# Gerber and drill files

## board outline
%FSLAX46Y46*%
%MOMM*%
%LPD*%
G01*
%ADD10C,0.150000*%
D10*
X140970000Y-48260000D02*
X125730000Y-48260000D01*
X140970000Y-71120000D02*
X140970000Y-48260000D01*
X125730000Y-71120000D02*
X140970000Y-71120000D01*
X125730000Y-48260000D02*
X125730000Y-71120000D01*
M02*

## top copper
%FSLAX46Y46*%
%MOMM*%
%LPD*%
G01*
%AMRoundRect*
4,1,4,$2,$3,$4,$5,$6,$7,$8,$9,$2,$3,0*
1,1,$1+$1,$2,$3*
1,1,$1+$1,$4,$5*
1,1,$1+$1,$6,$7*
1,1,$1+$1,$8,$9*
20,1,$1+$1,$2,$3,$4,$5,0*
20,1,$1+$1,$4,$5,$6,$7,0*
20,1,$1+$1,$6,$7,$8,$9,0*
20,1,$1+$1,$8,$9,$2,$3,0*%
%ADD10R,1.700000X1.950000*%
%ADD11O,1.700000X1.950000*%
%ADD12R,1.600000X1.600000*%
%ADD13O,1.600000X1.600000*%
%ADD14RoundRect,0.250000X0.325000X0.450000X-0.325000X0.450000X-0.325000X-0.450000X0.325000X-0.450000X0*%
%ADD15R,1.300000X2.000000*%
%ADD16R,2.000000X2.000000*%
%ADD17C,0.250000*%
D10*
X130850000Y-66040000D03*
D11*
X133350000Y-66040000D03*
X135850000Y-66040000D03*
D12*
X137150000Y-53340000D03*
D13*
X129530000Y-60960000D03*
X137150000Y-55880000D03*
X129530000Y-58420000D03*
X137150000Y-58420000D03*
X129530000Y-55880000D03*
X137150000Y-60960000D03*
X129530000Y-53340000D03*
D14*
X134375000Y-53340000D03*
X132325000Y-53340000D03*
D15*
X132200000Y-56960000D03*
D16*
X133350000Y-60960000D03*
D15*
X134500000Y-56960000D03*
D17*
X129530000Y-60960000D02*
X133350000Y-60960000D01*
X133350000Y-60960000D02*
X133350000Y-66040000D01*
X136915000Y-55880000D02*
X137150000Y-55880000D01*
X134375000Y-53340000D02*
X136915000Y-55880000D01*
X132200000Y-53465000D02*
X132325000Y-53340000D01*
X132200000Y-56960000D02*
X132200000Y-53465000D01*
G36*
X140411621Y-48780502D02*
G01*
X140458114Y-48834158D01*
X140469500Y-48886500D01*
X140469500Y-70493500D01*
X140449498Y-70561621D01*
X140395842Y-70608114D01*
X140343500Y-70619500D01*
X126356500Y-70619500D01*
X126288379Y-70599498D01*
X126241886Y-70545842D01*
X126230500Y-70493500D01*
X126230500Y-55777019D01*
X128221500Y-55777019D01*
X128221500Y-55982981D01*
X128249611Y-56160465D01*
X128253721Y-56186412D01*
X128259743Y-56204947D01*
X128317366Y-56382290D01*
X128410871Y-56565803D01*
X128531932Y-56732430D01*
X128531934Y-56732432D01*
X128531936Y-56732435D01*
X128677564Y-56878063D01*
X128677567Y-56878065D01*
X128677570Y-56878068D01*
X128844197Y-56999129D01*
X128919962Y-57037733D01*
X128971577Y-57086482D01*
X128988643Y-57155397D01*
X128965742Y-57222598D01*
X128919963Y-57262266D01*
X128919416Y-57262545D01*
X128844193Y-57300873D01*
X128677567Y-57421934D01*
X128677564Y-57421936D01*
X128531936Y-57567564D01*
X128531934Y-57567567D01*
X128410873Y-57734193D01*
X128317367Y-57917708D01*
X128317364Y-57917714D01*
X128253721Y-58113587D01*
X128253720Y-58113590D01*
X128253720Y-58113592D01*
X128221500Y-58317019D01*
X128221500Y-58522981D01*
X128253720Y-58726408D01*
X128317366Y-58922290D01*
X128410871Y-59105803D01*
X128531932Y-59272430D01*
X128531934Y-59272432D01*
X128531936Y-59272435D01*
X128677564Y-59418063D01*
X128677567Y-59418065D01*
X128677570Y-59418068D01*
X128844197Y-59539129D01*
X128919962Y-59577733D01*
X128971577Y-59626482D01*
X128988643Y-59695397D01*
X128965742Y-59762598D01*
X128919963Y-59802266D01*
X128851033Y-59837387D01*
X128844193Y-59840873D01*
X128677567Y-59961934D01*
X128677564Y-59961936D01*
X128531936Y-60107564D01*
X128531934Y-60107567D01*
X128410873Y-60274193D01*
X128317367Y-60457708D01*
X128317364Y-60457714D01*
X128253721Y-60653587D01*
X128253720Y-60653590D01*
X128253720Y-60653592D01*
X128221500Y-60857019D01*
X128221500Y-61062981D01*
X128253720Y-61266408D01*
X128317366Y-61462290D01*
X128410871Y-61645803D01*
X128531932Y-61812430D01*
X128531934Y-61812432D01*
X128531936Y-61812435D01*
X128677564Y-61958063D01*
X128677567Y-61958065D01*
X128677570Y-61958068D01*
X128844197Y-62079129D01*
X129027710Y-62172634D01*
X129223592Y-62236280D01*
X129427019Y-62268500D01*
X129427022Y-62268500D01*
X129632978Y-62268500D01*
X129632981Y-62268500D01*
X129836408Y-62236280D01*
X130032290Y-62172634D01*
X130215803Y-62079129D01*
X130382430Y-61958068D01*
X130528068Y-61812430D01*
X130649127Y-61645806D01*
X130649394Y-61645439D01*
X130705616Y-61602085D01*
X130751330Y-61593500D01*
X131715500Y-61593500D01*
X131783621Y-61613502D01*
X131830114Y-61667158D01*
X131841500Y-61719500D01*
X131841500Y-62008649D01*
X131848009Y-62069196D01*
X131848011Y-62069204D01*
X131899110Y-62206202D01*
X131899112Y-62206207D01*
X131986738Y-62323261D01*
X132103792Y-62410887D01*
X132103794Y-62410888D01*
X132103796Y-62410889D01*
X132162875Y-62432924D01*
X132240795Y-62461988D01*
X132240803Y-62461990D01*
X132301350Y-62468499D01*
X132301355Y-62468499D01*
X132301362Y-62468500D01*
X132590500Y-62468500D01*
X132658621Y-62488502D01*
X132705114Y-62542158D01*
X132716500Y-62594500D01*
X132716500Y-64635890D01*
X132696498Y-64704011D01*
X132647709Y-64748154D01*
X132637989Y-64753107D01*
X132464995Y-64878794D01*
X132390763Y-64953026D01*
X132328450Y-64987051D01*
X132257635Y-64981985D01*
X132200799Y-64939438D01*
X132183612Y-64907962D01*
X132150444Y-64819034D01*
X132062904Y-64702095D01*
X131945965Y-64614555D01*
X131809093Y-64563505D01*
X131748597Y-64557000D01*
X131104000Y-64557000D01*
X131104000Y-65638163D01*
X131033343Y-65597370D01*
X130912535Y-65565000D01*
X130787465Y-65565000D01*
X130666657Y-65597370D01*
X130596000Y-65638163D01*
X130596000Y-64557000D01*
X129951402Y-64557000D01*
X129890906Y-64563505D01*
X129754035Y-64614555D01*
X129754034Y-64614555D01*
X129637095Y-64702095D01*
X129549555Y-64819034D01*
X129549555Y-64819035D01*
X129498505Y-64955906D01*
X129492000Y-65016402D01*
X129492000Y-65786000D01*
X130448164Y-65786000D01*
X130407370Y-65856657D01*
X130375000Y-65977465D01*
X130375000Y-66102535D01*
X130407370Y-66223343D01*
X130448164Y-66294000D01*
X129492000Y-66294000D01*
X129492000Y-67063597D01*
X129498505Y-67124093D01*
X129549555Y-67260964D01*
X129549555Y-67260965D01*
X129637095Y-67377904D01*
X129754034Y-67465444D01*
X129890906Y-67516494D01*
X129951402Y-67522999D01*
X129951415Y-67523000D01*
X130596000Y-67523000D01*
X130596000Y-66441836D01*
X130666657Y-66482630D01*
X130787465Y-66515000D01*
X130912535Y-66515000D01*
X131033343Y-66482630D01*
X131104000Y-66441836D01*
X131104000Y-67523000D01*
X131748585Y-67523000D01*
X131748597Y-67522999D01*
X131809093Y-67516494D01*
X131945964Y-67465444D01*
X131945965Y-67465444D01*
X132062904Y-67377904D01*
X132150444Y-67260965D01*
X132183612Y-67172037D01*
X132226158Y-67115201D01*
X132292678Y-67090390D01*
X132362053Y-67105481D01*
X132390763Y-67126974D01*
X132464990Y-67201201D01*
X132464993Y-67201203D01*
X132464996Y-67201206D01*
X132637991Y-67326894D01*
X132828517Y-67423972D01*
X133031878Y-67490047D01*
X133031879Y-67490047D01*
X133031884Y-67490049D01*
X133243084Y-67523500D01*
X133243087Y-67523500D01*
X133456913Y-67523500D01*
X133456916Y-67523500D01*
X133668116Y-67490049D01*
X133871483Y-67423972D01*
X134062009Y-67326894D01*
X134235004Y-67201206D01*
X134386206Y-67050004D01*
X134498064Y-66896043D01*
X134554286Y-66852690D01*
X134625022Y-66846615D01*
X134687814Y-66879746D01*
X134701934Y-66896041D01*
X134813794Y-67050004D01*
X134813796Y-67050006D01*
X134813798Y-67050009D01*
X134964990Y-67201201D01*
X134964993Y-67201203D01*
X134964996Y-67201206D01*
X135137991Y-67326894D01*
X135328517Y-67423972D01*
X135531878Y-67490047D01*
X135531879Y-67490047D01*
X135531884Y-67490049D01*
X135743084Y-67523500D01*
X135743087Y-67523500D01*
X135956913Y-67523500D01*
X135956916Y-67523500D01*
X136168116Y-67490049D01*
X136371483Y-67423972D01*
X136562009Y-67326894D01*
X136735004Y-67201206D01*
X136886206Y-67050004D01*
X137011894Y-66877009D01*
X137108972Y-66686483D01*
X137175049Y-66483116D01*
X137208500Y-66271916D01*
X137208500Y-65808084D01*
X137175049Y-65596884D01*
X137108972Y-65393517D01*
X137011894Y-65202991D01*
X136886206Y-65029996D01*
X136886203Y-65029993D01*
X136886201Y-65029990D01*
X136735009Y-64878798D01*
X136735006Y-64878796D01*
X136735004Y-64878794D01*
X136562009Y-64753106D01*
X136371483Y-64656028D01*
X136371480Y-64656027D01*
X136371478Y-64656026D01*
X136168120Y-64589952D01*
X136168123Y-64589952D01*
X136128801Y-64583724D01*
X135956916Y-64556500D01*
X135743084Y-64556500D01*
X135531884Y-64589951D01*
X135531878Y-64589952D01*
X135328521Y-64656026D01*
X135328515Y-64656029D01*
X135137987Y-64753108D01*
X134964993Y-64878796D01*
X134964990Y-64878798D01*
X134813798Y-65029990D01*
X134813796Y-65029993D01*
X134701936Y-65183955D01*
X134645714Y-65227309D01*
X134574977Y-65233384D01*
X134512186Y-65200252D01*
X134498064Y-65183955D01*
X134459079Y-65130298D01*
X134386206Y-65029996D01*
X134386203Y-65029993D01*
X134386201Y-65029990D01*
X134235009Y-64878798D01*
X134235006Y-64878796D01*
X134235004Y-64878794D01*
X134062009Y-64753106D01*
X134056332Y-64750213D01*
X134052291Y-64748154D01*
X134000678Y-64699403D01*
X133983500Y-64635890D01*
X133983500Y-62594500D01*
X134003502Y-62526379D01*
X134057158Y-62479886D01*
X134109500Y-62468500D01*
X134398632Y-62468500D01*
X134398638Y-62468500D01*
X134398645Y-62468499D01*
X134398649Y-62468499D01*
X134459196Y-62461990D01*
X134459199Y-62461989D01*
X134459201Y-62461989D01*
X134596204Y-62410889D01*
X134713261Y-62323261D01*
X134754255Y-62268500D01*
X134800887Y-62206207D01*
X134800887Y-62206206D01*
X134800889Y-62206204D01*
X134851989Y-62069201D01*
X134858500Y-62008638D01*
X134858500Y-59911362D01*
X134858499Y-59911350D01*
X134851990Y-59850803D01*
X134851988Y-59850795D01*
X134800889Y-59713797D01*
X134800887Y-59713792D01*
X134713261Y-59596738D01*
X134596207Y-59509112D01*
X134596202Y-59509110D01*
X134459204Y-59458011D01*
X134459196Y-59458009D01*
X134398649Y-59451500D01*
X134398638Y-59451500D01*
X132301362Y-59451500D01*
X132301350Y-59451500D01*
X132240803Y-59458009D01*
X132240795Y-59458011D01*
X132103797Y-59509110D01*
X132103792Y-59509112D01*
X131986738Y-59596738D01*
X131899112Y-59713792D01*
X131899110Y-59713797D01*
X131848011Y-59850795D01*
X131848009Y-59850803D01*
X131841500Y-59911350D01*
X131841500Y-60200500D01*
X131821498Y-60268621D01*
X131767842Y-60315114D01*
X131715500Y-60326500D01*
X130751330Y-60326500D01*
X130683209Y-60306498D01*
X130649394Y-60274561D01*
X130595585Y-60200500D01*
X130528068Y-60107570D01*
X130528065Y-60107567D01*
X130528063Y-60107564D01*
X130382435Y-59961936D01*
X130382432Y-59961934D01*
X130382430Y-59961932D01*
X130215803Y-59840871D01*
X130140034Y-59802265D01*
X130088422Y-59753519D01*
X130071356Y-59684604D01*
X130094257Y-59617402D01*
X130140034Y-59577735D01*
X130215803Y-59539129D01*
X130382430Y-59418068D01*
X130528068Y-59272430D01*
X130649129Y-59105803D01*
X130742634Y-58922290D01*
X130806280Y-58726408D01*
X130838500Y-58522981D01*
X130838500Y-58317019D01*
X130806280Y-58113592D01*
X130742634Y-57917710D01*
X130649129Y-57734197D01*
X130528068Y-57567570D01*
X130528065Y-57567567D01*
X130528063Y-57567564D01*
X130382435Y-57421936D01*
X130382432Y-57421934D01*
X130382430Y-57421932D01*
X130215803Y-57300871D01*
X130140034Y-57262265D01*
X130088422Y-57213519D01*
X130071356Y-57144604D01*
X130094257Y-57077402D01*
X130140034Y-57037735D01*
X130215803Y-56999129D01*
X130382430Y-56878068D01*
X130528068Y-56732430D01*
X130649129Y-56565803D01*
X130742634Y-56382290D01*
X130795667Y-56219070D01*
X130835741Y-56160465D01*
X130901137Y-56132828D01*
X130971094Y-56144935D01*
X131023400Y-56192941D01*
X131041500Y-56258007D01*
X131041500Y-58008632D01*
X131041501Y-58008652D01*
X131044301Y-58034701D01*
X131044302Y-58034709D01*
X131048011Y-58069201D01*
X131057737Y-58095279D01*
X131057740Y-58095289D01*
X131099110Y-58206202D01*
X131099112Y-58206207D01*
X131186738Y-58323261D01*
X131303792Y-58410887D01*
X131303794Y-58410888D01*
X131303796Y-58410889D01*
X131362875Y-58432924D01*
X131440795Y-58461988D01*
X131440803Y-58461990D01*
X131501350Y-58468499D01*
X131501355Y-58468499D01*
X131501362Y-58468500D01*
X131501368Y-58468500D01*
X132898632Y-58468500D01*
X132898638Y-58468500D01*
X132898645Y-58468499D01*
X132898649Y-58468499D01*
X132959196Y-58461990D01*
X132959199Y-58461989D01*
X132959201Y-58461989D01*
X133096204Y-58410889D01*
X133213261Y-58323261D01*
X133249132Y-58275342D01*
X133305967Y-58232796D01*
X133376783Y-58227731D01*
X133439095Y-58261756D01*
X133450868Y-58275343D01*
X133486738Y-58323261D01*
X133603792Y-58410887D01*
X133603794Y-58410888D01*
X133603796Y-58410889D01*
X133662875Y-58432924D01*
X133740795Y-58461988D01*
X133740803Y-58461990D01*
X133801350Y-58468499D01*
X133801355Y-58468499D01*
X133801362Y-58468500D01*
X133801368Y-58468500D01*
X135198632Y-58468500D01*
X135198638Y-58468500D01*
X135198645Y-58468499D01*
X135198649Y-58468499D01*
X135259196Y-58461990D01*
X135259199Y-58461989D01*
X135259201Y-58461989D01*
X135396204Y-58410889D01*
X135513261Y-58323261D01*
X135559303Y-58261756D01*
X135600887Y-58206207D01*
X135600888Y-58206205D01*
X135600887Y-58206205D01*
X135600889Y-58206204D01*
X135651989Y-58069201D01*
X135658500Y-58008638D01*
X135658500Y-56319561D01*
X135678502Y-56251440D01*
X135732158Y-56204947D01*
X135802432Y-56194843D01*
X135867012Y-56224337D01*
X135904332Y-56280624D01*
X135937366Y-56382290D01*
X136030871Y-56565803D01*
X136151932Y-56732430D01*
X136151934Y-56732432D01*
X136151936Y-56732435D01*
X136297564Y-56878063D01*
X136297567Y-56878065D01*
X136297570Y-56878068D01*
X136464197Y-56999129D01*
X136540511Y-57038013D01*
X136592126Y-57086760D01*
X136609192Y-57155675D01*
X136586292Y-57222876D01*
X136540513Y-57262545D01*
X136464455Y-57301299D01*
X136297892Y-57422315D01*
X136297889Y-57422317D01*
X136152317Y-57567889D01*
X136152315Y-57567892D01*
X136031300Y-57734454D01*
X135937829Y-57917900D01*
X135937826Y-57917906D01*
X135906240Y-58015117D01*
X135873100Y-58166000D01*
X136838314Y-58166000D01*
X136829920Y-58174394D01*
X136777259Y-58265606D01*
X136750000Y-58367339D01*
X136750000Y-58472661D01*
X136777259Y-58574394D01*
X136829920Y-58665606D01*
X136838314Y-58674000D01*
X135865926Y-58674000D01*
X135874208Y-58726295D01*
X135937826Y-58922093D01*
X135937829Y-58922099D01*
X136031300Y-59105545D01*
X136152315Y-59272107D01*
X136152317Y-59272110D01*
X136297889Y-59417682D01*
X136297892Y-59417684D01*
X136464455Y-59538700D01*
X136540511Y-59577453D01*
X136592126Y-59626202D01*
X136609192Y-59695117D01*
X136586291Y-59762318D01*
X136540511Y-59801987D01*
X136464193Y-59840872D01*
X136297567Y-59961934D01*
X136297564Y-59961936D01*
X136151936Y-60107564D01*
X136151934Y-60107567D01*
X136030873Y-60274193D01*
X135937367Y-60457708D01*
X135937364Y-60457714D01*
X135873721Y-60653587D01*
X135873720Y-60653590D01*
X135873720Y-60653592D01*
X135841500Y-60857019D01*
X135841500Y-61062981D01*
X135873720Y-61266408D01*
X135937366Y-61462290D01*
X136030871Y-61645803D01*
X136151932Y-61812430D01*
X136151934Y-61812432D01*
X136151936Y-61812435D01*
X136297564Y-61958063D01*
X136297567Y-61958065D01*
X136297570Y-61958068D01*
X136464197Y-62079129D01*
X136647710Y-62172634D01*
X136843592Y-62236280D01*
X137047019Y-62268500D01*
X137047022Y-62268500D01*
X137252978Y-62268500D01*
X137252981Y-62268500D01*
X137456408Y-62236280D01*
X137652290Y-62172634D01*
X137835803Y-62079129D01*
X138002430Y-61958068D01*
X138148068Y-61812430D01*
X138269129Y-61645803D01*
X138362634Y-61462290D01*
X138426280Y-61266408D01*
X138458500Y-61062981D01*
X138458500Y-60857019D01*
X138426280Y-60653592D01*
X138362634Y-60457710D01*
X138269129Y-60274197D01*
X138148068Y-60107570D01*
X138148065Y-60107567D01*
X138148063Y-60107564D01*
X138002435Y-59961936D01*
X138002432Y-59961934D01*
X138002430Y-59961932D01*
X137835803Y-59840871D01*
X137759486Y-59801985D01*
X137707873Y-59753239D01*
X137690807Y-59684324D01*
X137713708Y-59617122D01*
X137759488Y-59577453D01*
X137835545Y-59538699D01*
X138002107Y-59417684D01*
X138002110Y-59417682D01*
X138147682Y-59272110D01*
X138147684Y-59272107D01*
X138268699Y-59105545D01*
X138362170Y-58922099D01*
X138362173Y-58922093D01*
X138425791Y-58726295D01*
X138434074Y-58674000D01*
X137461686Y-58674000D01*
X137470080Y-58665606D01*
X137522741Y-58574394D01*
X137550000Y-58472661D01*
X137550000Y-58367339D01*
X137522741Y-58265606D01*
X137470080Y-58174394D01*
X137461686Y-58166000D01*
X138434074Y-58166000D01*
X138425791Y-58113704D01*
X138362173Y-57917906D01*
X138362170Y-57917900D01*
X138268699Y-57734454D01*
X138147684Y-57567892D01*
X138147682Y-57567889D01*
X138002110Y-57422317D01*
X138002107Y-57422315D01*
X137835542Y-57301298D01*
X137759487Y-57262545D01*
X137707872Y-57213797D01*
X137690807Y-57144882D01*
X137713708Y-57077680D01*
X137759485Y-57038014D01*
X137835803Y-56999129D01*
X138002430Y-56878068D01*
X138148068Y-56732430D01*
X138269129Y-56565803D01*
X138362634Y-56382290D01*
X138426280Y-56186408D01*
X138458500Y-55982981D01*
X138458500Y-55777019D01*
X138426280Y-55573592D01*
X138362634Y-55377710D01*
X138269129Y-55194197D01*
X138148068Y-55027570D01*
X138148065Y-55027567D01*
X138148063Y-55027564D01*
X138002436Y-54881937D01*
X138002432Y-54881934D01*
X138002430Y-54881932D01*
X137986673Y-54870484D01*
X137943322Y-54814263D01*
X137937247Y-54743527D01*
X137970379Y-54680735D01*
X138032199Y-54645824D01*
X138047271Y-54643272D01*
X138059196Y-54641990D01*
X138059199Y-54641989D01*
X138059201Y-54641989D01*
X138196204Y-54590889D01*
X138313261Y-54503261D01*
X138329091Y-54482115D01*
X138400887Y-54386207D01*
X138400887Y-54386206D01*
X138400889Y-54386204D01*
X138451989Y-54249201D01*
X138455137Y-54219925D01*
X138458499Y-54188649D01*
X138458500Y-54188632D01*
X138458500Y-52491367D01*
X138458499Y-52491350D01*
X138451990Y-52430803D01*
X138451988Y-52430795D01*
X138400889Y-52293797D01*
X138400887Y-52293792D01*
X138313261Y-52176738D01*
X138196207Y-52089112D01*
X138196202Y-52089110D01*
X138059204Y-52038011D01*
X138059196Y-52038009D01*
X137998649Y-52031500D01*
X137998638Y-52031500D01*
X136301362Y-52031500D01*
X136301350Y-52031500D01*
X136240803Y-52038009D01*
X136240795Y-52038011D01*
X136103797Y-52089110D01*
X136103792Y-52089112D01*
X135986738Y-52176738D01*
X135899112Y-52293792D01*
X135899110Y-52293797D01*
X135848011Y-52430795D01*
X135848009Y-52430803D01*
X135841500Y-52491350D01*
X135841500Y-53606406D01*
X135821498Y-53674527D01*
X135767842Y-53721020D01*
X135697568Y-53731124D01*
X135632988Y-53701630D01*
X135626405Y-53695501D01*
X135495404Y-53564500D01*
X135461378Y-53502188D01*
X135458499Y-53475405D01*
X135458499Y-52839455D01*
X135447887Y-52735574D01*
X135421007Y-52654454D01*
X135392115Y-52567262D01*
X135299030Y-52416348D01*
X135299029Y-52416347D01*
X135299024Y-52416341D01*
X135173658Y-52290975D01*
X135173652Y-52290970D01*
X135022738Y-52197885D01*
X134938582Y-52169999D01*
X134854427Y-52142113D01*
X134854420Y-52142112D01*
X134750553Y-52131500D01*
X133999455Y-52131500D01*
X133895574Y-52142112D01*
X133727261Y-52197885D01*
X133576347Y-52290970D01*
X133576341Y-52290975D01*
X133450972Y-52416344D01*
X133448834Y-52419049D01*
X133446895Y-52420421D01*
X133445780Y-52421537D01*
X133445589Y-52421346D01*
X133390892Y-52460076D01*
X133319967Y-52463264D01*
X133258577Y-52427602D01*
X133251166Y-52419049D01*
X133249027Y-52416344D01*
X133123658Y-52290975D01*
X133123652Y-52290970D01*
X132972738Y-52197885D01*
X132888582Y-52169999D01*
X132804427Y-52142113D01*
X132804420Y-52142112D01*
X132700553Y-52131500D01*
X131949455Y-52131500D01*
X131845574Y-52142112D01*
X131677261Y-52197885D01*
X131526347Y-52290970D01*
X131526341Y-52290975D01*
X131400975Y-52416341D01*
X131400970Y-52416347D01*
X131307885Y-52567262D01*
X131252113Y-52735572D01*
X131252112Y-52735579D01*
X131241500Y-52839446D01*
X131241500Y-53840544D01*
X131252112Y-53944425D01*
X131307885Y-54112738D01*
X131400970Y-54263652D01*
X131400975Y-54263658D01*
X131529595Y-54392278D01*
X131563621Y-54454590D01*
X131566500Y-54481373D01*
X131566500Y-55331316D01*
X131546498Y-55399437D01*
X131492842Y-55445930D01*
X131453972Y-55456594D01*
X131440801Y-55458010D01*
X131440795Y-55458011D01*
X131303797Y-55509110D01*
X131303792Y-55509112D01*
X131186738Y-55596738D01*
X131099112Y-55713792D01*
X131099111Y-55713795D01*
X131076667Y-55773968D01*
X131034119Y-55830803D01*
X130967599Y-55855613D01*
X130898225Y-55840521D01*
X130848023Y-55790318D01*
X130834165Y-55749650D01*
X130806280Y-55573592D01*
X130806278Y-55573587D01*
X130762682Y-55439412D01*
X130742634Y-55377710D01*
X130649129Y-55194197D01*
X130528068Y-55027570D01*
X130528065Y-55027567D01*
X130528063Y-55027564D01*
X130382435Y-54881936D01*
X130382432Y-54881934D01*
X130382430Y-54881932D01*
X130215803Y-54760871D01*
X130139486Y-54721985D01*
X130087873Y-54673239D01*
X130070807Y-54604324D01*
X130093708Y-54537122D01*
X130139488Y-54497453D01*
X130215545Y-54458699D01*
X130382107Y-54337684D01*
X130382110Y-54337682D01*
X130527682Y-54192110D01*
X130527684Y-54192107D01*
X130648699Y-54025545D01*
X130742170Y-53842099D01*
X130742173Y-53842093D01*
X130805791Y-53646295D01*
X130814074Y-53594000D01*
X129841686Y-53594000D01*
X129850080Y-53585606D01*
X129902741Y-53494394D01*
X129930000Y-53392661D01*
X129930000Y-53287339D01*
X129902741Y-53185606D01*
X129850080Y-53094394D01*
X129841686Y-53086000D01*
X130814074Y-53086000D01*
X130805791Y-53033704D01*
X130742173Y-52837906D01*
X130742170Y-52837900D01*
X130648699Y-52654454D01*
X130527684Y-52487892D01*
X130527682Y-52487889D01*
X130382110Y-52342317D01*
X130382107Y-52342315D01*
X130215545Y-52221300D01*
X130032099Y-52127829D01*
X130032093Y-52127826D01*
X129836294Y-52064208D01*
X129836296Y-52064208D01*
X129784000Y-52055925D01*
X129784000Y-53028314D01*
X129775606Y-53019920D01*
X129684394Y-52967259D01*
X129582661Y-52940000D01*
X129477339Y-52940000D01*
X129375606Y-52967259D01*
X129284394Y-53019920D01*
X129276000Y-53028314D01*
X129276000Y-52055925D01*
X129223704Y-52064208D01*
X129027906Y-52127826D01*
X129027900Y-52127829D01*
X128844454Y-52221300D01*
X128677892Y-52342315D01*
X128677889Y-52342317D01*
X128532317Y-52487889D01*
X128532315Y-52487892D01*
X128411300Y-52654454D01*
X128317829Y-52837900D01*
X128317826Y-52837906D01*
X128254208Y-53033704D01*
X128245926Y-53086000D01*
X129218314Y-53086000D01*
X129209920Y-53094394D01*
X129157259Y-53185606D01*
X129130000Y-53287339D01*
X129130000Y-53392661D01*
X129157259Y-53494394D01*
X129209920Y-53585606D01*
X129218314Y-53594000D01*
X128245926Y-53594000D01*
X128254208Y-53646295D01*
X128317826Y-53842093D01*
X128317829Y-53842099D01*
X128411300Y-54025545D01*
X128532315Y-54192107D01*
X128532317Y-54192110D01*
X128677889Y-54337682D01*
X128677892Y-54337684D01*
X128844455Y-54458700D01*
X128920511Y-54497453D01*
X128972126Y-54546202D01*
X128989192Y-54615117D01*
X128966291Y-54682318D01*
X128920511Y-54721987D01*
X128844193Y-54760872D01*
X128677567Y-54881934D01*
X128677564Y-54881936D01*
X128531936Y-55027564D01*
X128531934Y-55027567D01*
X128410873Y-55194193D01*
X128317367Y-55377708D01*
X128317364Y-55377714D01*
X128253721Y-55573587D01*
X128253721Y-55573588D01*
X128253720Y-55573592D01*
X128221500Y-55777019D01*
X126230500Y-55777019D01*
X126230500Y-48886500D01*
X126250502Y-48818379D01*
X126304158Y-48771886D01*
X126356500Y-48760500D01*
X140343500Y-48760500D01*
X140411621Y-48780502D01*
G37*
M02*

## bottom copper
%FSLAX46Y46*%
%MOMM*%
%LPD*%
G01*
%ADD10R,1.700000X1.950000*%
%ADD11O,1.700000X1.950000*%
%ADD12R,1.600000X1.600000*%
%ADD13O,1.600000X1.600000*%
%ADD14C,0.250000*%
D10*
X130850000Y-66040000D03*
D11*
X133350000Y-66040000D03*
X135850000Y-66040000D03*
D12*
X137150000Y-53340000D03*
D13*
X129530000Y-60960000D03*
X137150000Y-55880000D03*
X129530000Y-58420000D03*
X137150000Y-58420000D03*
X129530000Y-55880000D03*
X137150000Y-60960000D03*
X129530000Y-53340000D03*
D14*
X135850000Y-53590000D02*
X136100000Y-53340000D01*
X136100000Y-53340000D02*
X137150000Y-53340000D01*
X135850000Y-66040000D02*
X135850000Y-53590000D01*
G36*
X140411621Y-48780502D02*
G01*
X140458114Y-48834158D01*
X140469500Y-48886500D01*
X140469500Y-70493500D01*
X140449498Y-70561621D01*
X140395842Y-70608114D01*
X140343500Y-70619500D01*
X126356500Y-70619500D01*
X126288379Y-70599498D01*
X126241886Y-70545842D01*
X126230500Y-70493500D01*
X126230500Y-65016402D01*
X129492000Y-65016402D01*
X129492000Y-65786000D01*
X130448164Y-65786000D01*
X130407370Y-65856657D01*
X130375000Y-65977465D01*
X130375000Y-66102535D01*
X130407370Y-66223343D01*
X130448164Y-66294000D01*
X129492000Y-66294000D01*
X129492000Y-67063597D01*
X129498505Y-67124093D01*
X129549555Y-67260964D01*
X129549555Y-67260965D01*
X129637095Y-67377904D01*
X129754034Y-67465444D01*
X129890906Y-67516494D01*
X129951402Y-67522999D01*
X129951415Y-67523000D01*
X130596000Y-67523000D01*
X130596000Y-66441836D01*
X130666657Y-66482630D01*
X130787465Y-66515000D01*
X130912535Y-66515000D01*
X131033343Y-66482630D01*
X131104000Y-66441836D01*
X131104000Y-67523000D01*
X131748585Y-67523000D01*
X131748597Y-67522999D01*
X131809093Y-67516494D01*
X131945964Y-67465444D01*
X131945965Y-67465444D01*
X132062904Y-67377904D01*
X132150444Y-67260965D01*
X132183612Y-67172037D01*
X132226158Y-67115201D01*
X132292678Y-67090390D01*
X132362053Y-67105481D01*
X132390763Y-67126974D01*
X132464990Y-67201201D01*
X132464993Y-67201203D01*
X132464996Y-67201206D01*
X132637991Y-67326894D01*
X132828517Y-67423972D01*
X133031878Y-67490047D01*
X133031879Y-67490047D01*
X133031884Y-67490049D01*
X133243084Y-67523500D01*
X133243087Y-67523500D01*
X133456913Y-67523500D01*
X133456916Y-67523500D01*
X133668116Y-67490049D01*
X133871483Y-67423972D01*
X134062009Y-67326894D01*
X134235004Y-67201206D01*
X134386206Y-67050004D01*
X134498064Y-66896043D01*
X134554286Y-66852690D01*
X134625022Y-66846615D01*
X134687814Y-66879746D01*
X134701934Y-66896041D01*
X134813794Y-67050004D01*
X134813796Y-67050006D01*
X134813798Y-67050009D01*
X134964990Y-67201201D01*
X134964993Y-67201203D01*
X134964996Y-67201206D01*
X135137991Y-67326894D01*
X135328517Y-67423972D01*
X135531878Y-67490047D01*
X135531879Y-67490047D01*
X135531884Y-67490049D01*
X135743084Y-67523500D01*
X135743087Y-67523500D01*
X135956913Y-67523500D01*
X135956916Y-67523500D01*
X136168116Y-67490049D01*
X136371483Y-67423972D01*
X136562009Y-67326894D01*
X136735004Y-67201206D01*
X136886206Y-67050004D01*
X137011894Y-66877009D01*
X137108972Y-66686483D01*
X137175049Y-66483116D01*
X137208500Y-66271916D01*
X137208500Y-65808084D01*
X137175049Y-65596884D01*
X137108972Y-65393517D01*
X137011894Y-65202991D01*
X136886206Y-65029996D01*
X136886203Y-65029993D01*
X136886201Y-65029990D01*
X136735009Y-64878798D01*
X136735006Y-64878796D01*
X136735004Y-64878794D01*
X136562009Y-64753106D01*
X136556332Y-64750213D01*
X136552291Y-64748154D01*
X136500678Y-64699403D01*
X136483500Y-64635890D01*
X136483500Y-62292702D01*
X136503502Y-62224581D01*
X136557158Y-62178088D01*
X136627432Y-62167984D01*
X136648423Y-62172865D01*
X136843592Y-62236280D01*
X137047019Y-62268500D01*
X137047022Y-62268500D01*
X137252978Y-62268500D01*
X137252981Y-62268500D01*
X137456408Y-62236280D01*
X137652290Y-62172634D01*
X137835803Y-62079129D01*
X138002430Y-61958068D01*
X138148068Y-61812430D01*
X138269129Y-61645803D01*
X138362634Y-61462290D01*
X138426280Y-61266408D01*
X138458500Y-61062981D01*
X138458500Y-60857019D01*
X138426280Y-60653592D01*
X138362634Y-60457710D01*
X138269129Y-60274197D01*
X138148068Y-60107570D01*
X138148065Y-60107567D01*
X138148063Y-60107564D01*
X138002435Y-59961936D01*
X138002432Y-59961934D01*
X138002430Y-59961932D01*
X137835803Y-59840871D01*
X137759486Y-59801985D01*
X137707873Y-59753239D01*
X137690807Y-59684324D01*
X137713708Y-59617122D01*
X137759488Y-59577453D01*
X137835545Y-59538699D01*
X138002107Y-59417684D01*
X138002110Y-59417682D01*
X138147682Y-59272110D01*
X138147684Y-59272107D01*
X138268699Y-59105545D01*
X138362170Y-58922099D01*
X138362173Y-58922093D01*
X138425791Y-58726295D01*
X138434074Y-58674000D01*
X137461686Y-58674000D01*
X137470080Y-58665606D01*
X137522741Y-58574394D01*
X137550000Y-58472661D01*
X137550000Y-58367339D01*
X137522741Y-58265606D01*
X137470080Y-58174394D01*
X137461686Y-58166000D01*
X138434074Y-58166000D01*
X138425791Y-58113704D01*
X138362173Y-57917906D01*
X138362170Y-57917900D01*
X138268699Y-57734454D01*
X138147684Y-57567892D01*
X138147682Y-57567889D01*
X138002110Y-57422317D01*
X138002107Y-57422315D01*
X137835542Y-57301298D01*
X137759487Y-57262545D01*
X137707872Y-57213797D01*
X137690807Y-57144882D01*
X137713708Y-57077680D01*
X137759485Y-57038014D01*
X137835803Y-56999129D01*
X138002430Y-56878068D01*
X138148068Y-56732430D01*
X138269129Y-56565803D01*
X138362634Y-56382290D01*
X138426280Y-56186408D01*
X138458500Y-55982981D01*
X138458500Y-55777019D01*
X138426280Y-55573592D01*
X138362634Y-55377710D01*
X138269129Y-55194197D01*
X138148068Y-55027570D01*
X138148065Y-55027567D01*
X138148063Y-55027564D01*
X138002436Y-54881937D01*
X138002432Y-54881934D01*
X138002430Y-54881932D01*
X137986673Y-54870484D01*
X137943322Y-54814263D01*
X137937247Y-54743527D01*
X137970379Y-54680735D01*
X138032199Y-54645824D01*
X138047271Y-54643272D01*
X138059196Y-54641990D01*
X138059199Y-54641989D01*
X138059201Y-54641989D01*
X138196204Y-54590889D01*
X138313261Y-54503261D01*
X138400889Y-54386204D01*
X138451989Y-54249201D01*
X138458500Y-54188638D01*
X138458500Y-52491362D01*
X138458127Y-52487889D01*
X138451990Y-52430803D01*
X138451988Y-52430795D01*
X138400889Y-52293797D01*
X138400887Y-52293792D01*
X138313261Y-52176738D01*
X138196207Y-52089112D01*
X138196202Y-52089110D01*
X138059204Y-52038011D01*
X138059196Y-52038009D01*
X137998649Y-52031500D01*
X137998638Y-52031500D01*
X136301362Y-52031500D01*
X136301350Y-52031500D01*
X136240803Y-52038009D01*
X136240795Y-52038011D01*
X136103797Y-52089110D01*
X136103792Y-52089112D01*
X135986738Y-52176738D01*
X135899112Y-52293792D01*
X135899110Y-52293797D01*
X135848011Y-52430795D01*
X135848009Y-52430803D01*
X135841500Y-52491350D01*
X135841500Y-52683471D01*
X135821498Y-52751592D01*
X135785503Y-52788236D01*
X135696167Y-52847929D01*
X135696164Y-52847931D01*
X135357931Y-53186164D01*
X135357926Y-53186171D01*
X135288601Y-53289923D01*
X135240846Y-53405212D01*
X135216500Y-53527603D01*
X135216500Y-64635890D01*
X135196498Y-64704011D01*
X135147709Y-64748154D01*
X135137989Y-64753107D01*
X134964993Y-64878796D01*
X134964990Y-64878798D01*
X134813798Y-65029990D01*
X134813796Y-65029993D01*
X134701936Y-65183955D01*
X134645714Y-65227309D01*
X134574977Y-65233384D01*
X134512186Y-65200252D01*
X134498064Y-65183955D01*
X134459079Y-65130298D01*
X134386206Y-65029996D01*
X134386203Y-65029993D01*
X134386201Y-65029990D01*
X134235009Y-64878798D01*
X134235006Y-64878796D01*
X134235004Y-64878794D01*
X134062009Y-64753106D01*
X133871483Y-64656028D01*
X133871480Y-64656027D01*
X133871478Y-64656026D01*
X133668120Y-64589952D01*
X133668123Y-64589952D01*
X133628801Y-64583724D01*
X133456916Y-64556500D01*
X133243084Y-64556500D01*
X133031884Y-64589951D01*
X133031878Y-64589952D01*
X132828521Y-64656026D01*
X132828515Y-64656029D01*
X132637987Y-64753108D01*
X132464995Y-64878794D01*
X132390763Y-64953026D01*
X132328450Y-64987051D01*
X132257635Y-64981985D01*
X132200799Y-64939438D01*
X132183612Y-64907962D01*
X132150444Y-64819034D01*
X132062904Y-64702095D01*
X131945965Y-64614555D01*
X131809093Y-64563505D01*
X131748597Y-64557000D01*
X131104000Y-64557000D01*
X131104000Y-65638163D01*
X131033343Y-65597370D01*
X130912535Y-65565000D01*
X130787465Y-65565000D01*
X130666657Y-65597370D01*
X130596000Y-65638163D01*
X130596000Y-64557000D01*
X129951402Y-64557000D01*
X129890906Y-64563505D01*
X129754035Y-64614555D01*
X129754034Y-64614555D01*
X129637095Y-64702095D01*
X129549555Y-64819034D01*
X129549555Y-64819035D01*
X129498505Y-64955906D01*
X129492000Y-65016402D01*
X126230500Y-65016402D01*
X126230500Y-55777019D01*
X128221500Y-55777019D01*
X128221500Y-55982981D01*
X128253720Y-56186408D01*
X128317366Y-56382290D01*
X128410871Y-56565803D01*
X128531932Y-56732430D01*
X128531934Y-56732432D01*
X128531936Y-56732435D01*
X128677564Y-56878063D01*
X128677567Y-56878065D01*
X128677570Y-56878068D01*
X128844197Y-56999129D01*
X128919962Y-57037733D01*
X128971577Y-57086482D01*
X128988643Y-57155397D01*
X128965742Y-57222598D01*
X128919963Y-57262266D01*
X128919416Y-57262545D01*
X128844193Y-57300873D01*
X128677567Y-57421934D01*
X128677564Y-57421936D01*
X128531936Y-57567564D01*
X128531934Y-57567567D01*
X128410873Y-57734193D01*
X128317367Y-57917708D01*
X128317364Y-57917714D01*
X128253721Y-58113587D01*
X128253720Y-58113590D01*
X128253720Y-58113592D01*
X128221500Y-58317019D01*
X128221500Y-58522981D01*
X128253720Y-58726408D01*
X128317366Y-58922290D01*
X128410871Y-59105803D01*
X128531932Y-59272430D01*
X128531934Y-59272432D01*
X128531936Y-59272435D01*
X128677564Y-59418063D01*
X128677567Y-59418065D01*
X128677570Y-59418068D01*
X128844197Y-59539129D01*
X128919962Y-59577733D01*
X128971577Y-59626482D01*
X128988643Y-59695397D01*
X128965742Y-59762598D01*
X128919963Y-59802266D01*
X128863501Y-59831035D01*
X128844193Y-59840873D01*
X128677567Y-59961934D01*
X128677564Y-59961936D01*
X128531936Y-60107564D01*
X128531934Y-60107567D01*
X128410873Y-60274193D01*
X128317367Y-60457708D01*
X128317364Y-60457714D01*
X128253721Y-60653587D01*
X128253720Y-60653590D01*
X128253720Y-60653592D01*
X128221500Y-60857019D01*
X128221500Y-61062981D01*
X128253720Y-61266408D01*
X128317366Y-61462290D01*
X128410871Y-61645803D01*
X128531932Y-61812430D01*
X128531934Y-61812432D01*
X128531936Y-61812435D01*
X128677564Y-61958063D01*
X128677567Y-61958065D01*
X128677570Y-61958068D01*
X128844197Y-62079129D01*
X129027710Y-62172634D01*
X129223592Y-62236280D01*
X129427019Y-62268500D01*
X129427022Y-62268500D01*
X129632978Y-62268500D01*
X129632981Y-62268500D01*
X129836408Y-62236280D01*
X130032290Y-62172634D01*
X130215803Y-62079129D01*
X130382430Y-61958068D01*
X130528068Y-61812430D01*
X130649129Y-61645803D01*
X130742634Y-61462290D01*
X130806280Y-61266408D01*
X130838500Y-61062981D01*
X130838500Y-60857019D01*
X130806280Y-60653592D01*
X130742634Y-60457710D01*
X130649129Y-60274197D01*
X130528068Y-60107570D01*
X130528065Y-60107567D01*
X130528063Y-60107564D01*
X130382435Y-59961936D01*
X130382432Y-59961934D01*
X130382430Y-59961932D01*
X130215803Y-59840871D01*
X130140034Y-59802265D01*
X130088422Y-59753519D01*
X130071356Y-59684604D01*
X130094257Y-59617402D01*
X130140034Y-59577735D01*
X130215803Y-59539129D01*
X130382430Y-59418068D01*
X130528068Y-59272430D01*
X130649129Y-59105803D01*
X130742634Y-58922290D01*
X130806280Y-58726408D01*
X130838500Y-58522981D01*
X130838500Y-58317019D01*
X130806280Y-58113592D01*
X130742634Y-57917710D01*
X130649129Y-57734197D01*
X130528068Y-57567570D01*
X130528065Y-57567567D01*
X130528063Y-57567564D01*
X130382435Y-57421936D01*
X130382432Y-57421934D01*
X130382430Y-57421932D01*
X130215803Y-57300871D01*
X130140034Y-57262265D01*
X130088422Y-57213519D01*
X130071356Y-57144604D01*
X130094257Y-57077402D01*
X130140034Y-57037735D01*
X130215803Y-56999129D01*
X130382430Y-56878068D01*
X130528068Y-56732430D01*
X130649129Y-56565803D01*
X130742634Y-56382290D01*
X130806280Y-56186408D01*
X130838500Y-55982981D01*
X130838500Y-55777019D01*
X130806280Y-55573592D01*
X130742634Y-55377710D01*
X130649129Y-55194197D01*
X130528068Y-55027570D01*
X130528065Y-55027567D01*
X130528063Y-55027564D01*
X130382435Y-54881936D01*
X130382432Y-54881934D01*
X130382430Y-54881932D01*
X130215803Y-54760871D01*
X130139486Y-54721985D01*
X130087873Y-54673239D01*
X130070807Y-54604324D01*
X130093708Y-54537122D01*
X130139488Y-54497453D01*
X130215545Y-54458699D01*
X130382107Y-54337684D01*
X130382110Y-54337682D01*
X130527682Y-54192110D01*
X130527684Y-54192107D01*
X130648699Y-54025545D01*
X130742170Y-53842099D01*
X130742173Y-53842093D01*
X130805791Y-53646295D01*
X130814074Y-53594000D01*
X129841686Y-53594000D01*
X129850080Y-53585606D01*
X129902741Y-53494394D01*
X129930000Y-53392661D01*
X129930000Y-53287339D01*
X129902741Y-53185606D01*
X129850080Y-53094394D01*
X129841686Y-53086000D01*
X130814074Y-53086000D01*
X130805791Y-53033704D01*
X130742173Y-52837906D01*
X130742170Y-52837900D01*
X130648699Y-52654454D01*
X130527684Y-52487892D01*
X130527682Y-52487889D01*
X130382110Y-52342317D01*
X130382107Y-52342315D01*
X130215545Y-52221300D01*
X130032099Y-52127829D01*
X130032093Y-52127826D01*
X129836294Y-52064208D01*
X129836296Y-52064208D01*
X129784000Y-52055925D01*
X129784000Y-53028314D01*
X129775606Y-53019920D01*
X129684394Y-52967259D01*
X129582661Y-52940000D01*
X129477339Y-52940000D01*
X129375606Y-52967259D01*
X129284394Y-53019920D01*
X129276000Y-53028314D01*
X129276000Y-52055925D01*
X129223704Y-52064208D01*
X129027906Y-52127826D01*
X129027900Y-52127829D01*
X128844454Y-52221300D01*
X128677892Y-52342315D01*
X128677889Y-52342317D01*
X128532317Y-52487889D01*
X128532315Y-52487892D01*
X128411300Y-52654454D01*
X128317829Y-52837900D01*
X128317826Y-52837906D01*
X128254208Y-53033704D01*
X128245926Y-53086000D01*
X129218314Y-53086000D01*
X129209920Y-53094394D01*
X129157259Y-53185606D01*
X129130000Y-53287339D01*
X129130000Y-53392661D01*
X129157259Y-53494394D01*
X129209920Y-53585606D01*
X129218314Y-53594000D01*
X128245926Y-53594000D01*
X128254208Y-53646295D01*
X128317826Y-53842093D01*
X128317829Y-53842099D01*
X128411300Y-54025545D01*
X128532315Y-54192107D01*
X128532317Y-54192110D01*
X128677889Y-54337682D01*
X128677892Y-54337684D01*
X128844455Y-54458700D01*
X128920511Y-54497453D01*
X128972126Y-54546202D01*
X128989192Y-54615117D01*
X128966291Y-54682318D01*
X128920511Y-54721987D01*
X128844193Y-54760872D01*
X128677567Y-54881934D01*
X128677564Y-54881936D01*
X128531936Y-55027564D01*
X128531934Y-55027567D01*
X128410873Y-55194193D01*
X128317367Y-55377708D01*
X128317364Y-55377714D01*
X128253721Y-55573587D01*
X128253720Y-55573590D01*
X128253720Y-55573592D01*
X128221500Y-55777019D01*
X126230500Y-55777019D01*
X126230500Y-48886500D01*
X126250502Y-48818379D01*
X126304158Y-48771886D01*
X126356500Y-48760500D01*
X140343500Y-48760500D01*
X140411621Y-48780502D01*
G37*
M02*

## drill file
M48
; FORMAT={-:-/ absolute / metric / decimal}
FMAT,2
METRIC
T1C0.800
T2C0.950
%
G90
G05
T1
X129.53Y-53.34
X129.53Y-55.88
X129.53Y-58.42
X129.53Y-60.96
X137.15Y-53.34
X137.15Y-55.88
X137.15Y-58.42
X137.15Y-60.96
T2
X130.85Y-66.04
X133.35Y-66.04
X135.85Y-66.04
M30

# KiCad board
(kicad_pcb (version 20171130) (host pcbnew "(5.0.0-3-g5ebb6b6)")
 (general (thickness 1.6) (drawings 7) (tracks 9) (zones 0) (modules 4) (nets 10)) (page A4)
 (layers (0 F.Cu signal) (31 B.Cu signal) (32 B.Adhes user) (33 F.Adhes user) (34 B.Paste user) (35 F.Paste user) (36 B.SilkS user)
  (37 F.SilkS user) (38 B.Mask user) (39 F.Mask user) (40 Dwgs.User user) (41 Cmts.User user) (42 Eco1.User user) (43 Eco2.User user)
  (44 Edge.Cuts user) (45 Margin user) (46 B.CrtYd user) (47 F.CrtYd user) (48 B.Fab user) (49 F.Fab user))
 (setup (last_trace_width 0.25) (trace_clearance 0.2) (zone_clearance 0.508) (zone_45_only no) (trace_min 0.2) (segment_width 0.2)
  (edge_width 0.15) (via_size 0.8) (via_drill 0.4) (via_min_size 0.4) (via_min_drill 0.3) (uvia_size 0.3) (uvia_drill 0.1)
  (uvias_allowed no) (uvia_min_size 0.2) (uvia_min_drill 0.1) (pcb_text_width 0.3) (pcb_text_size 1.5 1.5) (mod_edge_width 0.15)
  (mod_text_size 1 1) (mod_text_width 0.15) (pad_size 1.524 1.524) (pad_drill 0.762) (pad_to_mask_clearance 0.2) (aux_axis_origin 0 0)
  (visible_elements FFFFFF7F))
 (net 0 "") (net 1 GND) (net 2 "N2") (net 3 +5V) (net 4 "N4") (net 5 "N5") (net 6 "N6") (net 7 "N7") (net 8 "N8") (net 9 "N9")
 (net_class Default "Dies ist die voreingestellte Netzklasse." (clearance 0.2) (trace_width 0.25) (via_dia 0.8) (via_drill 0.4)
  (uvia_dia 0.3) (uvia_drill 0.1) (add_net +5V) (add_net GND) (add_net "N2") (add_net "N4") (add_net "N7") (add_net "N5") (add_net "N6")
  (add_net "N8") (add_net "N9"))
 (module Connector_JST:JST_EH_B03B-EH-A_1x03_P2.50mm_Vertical (layer F.Cu) (at 130.85 66.04)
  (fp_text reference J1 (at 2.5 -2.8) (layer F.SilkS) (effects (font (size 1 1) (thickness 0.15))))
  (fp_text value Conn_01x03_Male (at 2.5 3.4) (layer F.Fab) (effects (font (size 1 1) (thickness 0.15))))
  (pad 1 thru_hole rect (at 0 0) (size 1.7 1.95) (drill 0.95) (layers *.Cu *.Mask) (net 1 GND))
  (pad 2 thru_hole oval (at 2.5 0) (size 1.7 1.95) (drill 0.95) (layers *.Cu *.Mask) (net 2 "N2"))
  (pad 3 thru_hole oval (at 5 0) (size 1.7 1.95) (drill 0.95) (layers *.Cu *.Mask) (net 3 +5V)))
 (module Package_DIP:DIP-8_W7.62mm (layer B.Cu) (at 137.15 53.34 180)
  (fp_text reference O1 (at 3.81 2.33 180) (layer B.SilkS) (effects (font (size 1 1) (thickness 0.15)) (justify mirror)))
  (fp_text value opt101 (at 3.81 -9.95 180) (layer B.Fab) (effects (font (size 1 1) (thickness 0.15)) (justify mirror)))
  (pad 1 thru_hole rect (at 0 0 180) (size 1.6 1.6) (drill 0.8) (layers *.Cu *.Mask) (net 3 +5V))
  (pad 5 thru_hole oval (at 7.62 -7.62 180) (size 1.6 1.6) (drill 0.8) (layers *.Cu *.Mask) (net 2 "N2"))
  (pad 2 thru_hole oval (at 0 -2.54 180) (size 1.6 1.6) (drill 0.8) (layers *.Cu *.Mask) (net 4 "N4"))
  (pad 6 thru_hole oval (at 7.62 -5.08 180) (size 1.6 1.6) (drill 0.8) (layers *.Cu *.Mask) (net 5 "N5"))
  (pad 3 thru_hole oval (at 0 -5.08 180) (size 1.6 1.6) (drill 0.8) (layers *.Cu *.Mask) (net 1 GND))
  (pad 7 thru_hole oval (at 7.62 -2.54 180) (size 1.6 1.6) (drill 0.8) (layers *.Cu *.Mask) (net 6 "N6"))
  (pad 4 thru_hole oval (at 0 -7.62 180) (size 1.6 1.6) (drill 0.8) (layers *.Cu *.Mask) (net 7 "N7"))
  (pad 8 thru_hole oval (at 7.62 0 180) (size 1.6 1.6) (drill 0.8) (layers *.Cu *.Mask) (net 1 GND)))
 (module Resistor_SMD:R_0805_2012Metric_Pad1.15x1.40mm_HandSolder (layer F.Cu) (at 133.35 53.34 180)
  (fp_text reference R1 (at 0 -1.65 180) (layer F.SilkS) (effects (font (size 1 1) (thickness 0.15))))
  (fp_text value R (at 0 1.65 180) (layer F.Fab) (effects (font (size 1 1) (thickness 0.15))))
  (pad 1 smd roundrect (at -1.025 0 180) (size 1.15 1.4) (layers F.Cu F.Paste F.Mask) (roundrect_rratio 0.217391) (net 4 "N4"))
  (pad 2 smd roundrect (at 1.025 0 180) (size 1.15 1.4) (layers F.Cu F.Paste F.Mask) (roundrect_rratio 0.217391) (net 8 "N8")))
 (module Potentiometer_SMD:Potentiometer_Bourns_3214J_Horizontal (layer F.Cu) (at 133.35 58.96 90)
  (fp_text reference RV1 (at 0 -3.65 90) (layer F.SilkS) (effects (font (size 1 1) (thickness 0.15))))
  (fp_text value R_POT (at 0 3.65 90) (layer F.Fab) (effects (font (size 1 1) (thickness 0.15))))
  (pad 1 smd rect (at 2 -1.15 90) (size 2 1.3) (layers F.Cu F.Paste F.Mask) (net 8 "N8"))
  (pad 2 smd rect (at -2 0 90) (size 2 2) (layers F.Cu F.Paste F.Mask) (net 2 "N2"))
  (pad 3 smd rect (at 2 1.15 90) (size 2 1.3) (layers F.Cu F.Paste F.Mask) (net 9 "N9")))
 (gr_line (start 140.97 48.26) (end 125.73 48.26) (layer Edge.Cuts) (width 0.15))
 (gr_line (start 140.97 71.12) (end 140.97 48.26) (layer Edge.Cuts) (width 0.15))
 (gr_line (start 125.73 71.12) (end 140.97 71.12) (layer Edge.Cuts) (width 0.15))
 (gr_line (start 125.73 48.26) (end 125.73 71.12) (layer Edge.Cuts) (width 0.15))
 (segment (start 129.53 60.96) (end 133.35 60.96) (width 0.25) (layer F.Cu) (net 2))
 (segment (start 133.35 60.96) (end 133.35 66.04) (width 0.25) (layer F.Cu) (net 2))
 (segment (start 135.85 53.59) (end 136.1 53.34) (width 0.25) (layer B.Cu) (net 3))
 (segment (start 136.1 53.34) (end 137.15 53.34) (width 0.25) (layer B.Cu) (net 3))
 (segment (start 135.85 66.04) (end 135.85 53.59) (width 0.25) (layer B.Cu) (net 3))
 (segment (start 136.915 55.88) (end 137.15 55.88) (width 0.25) (layer F.Cu) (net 4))
 (segment (start 134.375 53.34) (end 136.915 55.88) (width 0.25) (layer F.Cu) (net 4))
 (segment (start 132.2 53.465) (end 132.325 53.34) (width 0.25) (layer F.Cu) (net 8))
 (segment (start 132.2 56.96) (end 132.2 53.465) (width 0.25) (layer F.Cu) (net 8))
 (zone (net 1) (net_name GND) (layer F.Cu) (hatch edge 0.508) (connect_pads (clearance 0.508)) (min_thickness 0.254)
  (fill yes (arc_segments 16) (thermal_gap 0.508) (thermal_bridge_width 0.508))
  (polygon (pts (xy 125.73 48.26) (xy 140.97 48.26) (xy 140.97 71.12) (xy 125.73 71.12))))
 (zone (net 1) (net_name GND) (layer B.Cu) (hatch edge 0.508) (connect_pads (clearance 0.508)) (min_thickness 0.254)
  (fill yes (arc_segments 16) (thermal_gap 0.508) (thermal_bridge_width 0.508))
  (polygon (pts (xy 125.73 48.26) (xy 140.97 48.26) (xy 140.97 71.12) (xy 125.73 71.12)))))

